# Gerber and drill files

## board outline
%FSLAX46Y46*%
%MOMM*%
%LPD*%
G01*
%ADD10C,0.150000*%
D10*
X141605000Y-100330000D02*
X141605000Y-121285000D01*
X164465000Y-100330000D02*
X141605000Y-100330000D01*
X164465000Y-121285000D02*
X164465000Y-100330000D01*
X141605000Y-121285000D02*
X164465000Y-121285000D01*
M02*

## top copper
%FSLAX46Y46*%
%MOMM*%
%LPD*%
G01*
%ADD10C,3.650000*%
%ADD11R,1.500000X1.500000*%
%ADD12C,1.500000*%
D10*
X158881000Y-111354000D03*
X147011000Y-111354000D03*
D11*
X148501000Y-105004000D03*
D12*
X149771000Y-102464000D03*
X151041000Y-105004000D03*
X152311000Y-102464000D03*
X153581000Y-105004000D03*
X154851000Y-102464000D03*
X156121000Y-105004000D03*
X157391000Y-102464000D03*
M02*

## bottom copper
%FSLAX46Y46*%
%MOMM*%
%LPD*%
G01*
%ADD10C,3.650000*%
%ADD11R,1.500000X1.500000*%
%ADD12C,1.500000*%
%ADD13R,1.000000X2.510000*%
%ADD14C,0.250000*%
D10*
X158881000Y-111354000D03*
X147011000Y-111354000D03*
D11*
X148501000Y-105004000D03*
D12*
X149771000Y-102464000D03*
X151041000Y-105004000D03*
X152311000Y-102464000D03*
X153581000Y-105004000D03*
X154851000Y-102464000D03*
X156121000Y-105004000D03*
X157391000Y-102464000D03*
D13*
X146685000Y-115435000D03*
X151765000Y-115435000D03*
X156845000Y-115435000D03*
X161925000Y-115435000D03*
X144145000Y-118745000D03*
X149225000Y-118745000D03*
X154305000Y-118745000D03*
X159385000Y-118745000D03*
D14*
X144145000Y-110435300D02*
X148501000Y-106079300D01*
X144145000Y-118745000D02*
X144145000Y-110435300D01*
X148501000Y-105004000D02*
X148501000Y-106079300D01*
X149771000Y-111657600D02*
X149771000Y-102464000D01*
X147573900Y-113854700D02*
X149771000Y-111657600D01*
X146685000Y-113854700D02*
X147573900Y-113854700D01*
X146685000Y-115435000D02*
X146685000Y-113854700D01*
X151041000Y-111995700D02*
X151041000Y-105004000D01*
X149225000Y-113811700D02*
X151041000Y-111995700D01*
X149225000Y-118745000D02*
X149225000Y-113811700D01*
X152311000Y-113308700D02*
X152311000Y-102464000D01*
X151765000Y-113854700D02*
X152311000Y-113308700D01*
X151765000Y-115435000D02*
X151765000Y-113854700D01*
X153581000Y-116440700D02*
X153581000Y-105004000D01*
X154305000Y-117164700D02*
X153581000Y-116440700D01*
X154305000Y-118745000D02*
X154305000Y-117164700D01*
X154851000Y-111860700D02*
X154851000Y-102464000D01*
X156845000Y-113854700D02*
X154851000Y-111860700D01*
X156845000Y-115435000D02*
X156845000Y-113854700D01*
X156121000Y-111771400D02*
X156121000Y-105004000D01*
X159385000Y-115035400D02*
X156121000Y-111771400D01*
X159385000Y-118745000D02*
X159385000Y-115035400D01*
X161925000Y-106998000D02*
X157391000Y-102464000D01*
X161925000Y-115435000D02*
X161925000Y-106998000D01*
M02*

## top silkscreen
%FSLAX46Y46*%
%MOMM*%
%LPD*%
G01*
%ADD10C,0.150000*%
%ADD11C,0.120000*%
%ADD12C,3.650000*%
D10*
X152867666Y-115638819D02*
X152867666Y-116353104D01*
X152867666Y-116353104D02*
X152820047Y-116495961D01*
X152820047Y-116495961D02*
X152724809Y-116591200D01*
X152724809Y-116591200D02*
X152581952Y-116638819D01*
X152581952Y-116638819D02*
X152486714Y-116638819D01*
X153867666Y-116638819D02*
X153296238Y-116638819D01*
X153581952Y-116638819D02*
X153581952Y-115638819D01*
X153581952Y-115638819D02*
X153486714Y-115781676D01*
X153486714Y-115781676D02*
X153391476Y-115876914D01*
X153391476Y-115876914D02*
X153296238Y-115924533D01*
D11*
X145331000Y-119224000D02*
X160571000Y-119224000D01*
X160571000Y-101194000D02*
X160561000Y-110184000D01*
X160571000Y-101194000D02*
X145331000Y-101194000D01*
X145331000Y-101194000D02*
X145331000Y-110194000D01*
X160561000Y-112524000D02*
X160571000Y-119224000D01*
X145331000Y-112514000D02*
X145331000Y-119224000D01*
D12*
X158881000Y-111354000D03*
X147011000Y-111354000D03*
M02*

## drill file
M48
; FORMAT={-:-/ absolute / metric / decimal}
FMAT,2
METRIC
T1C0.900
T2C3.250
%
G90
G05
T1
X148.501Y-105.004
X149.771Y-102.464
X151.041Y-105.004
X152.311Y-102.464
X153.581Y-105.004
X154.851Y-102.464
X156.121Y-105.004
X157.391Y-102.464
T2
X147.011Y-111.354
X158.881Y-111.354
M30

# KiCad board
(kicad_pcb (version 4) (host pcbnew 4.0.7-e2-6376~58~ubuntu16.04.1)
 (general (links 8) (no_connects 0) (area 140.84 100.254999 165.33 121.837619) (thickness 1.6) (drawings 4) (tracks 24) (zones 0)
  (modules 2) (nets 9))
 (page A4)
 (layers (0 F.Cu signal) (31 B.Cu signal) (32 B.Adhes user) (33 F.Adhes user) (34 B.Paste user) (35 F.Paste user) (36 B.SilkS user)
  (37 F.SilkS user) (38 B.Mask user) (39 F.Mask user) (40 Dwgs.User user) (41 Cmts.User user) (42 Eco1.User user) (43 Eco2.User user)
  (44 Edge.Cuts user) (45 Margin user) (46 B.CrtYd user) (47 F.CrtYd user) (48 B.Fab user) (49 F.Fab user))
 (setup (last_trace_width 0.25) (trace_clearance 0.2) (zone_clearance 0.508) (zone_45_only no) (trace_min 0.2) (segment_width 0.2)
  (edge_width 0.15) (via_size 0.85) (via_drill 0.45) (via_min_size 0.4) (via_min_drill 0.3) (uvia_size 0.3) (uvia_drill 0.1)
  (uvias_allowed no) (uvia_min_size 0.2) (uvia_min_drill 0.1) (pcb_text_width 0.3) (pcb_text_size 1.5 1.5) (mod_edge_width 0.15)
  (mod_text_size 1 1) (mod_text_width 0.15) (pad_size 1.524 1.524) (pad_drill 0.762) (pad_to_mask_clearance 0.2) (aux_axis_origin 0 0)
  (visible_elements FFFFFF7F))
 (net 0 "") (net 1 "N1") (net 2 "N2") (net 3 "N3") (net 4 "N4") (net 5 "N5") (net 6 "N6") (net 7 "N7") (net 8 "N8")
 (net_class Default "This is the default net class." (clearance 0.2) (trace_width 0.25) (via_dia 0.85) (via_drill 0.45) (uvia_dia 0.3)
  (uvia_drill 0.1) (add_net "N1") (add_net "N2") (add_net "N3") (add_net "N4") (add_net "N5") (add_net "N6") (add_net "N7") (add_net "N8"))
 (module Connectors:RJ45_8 (layer F.Cu) (at 148.501 105.004)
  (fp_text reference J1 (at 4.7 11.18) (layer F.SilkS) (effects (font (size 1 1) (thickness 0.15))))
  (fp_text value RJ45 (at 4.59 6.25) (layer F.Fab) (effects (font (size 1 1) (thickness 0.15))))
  (fp_line (start -3.17 14.22) (end 12.07 14.22) (layer F.SilkS) (width 0.12))
  (fp_line (start 12.07 -3.81) (end 12.06 5.18) (layer F.SilkS) (width 0.12))
  (fp_line (start 12.07 -3.81) (end -3.17 -3.81) (layer F.SilkS) (width 0.12))
  (fp_line (start -3.17 -3.81) (end -3.17 5.19) (layer F.SilkS) (width 0.12))
  (fp_line (start 12.06 7.52) (end 12.07 14.22) (layer F.SilkS) (width 0.12))
  (fp_line (start -3.17 7.51) (end -3.17 14.22) (layer F.SilkS) (width 0.12))
  (pad Hole np_thru_hole circle (at 10.38 6.35) (size 3.65 3.65) (drill 3.25) (layers *.Cu *.SilkS *.Mask))
  (pad Hole np_thru_hole circle (at -1.49 6.35) (size 3.65 3.65) (drill 3.25) (layers *.Cu *.SilkS *.Mask))
  (pad 1 thru_hole rect (at 0 0) (size 1.5 1.5) (drill 0.9) (layers *.Cu *.Mask) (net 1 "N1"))
  (pad 2 thru_hole circle (at 1.27 -2.54) (size 1.5 1.5) (drill 0.9) (layers *.Cu *.Mask) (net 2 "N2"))
  (pad 3 thru_hole circle (at 2.54 0) (size 1.5 1.5) (drill 0.9) (layers *.Cu *.Mask) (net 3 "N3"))
  (pad 4 thru_hole circle (at 3.81 -2.54) (size 1.5 1.5) (drill 0.9) (layers *.Cu *.Mask) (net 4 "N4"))
  (pad 5 thru_hole circle (at 5.08 0) (size 1.5 1.5) (drill 0.9) (layers *.Cu *.Mask) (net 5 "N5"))
  (pad 6 thru_hole circle (at 6.35 -2.54) (size 1.5 1.5) (drill 0.9) (layers *.Cu *.Mask) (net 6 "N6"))
  (pad 7 thru_hole circle (at 7.62 0) (size 1.5 1.5) (drill 0.9) (layers *.Cu *.Mask) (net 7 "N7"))
  (pad 8 thru_hole circle (at 8.89 -2.54) (size 1.5 1.5) (drill 0.9) (layers *.Cu *.Mask) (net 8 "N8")))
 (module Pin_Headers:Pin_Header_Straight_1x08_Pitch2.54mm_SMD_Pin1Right (layer B.Cu) (at 153.035 117.09 270)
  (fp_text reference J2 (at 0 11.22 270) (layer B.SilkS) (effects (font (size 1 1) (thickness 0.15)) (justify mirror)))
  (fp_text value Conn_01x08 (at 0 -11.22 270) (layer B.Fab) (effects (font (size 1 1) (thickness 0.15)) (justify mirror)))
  (pad 2 smd rect (at -1.655 6.35 270) (size 2.51 1) (layers B.Cu B.Paste B.Mask) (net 2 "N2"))
  (pad 4 smd rect (at -1.655 1.27 270) (size 2.51 1) (layers B.Cu B.Paste B.Mask) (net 4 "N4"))
  (pad 6 smd rect (at -1.655 -3.81 270) (size 2.51 1) (layers B.Cu B.Paste B.Mask) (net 6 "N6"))
  (pad 8 smd rect (at -1.655 -8.89 270) (size 2.51 1) (layers B.Cu B.Paste B.Mask) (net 8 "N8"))
  (pad 1 smd rect (at 1.655 8.89 270) (size 2.51 1) (layers B.Cu B.Paste B.Mask) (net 1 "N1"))
  (pad 3 smd rect (at 1.655 3.81 270) (size 2.51 1) (layers B.Cu B.Paste B.Mask) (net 3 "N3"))
  (pad 5 smd rect (at 1.655 -1.27 270) (size 2.51 1) (layers B.Cu B.Paste B.Mask) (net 5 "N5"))
  (pad 7 smd rect (at 1.655 -6.35 270) (size 2.51 1) (layers B.Cu B.Paste B.Mask) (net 7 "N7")))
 (gr_line (start 141.605 100.33) (end 141.605 121.285) (layer Edge.Cuts) (width 0.15))
 (gr_line (start 164.465 100.33) (end 141.605 100.33) (layer Edge.Cuts) (width 0.15))
 (gr_line (start 164.465 121.285) (end 164.465 100.33) (layer Edge.Cuts) (width 0.15))
 (gr_line (start 141.605 121.285) (end 164.465 121.285) (layer Edge.Cuts) (width 0.15))
 (segment (start 144.145 110.4353) (end 148.501 106.0793) (width 0.25) (layer B.Cu) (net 1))
 (segment (start 144.145 118.745) (end 144.145 110.4353) (width 0.25) (layer B.Cu) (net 1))
 (segment (start 148.501 105.004) (end 148.501 106.0793) (width 0.25) (layer B.Cu) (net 1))
 (segment (start 149.771 111.6576) (end 149.771 102.464) (width 0.25) (layer B.Cu) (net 2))
 (segment (start 147.5739 113.8547) (end 149.771 111.6576) (width 0.25) (layer B.Cu) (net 2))
 (segment (start 146.685 113.8547) (end 147.5739 113.8547) (width 0.25) (layer B.Cu) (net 2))
 (segment (start 146.685 115.435) (end 146.685 113.8547) (width 0.25) (layer B.Cu) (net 2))
 (segment (start 151.041 111.9957) (end 151.041 105.004) (width 0.25) (layer B.Cu) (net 3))
 (segment (start 149.225 113.8117) (end 151.041 111.9957) (width 0.25) (layer B.Cu) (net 3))
 (segment (start 149.225 118.745) (end 149.225 113.8117) (width 0.25) (layer B.Cu) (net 3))
 (segment (start 152.311 113.3087) (end 152.311 102.464) (width 0.25) (layer B.Cu) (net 4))
 (segment (start 151.765 113.8547) (end 152.311 113.3087) (width 0.25) (layer B.Cu) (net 4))
 (segment (start 151.765 115.435) (end 151.765 113.8547) (width 0.25) (layer B.Cu) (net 4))
 (segment (start 153.581 116.4407) (end 153.581 105.004) (width 0.25) (layer B.Cu) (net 5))
 (segment (start 154.305 117.1647) (end 153.581 116.4407) (width 0.25) (layer B.Cu) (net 5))
 (segment (start 154.305 118.745) (end 154.305 117.1647) (width 0.25) (layer B.Cu) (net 5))
 (segment (start 154.851 111.8607) (end 154.851 102.464) (width 0.25) (layer B.Cu) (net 6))
 (segment (start 156.845 113.8547) (end 154.851 111.8607) (width 0.25) (layer B.Cu) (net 6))
 (segment (start 156.845 115.435) (end 156.845 113.8547) (width 0.25) (layer B.Cu) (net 6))
 (segment (start 156.121 111.7714) (end 156.121 105.004) (width 0.25) (layer B.Cu) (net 7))
 (segment (start 159.385 115.0354) (end 156.121 111.7714) (width 0.25) (layer B.Cu) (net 7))
 (segment (start 159.385 118.745) (end 159.385 115.0354) (width 0.25) (layer B.Cu) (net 7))
 (segment (start 161.925 106.998) (end 157.391 102.464) (width 0.25) (layer B.Cu) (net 8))
 (segment (start 161.925 115.435) (end 161.925 106.998) (width 0.25) (layer B.Cu) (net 8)))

